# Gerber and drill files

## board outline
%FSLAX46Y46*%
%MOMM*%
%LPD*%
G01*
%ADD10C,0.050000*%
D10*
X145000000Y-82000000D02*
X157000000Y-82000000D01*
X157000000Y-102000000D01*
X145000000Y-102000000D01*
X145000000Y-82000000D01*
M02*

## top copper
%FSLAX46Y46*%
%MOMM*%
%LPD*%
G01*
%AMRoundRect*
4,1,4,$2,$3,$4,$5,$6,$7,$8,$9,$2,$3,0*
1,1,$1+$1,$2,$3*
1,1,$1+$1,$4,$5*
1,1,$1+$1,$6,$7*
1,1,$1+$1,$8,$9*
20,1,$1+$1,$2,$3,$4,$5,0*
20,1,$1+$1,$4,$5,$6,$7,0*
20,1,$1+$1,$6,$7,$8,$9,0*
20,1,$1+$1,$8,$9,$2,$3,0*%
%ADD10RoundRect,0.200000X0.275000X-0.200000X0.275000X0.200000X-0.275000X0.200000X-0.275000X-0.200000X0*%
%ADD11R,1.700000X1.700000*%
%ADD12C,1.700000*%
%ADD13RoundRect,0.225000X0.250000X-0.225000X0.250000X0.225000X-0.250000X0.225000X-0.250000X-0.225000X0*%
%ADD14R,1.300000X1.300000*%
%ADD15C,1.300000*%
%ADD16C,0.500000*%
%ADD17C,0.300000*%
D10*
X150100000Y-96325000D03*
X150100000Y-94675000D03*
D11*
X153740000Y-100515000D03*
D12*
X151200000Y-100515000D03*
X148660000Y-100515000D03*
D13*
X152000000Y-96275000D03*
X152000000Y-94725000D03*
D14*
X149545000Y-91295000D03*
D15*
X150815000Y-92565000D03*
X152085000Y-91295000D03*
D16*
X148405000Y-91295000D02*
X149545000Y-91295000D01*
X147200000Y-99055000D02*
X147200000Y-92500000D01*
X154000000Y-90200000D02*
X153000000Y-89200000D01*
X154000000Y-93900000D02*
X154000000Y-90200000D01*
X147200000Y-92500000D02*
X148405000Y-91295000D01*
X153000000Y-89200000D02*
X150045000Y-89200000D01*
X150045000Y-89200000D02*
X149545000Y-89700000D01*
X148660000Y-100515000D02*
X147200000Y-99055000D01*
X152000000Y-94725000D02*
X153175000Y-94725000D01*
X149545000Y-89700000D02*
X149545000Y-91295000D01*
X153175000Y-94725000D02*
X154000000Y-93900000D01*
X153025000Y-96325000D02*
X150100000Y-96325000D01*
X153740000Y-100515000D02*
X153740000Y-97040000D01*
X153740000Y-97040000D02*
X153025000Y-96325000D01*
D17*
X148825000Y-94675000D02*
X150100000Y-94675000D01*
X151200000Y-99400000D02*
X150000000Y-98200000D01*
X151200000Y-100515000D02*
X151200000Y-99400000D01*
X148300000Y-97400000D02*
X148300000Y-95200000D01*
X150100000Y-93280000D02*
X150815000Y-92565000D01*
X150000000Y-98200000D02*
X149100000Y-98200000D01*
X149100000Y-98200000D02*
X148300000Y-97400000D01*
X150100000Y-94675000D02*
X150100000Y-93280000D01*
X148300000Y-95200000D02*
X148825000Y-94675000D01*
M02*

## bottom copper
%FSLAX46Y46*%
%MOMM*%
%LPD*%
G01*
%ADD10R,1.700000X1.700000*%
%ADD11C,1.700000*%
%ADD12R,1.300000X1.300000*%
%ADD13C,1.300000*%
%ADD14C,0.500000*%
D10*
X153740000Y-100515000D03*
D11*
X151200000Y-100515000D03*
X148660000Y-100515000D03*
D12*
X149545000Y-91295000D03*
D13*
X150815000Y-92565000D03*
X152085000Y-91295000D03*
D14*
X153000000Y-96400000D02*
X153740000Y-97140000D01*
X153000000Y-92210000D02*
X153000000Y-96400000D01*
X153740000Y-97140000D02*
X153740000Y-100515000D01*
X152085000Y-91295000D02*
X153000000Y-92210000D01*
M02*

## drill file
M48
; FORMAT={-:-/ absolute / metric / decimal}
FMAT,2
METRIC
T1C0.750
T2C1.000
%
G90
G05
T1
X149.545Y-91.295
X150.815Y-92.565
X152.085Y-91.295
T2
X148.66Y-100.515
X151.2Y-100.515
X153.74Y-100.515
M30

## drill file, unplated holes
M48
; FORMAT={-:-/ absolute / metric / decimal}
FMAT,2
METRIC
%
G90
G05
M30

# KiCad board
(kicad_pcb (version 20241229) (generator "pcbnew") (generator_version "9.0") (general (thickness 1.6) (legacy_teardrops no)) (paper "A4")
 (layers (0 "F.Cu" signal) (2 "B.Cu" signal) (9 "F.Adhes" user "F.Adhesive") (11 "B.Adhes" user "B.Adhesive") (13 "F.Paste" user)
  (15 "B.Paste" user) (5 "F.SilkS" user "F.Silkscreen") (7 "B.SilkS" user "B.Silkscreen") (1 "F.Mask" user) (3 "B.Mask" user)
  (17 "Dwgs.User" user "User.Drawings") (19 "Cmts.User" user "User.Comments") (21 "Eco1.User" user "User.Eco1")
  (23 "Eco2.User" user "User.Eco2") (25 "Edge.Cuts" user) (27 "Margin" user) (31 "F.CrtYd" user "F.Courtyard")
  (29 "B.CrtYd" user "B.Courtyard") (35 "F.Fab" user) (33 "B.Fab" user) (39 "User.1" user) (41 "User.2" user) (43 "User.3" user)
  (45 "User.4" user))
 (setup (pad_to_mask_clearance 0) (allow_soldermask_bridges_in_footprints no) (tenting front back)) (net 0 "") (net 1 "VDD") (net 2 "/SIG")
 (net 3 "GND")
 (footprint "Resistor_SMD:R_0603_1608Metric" (layer "F.Cu") (at 150.1 95.5 90)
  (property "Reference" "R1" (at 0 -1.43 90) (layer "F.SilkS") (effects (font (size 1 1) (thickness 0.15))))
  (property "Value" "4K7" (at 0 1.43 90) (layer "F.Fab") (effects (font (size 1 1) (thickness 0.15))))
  (pad "1" smd roundrect (at -0.825 0 90) (size 0.8 0.95) (layers "F.Cu" "F.Mask" "F.Paste") (roundrect_rratio 0.25) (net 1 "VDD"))
  (pad "2" smd roundrect (at 0.825 0 90) (size 0.8 0.95) (layers "F.Cu" "F.Mask" "F.Paste") (roundrect_rratio 0.25) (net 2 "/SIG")))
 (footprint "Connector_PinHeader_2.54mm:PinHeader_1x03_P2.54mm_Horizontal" (layer "F.Cu") (at 153.74 100.515 -90)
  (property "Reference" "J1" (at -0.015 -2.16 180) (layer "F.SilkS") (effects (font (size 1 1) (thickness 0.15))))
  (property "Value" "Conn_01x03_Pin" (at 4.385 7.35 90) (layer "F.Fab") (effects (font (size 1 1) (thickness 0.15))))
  (pad "1" thru_hole rect (at 0 0 270) (size 1.7 1.7) (drill 1) (layers "*.Cu" "*.Mask") (remove_unused_layers no) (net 1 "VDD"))
  (pad "2" thru_hole circle (at 0 2.54 270) (size 1.7 1.7) (drill 1) (layers "*.Cu" "*.Mask") (remove_unused_layers no) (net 2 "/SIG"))
  (pad "3" thru_hole circle (at 0 5.08 270) (size 1.7 1.7) (drill 1) (layers "*.Cu" "*.Mask") (remove_unused_layers no) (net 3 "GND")))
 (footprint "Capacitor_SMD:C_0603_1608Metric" (layer "F.Cu") (at 152 95.5 90)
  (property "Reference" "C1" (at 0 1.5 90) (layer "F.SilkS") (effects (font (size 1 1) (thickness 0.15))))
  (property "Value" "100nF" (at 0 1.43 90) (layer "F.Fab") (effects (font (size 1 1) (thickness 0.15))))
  (pad "1" smd roundrect (at -0.775 0 90) (size 0.9 0.95) (layers "F.Cu" "F.Mask" "F.Paste") (roundrect_rratio 0.25) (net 1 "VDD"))
  (pad "2" smd roundrect (at 0.775 0 90) (size 0.9 0.95) (layers "F.Cu" "F.Mask" "F.Paste") (roundrect_rratio 0.25) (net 3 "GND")))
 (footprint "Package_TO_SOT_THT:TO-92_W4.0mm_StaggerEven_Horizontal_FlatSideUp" (layer "F.Cu") (at 149.545 91.295)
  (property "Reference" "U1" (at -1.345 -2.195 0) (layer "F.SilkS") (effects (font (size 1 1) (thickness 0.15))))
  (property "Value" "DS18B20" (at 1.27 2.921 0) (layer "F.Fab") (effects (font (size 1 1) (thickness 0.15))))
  (pad "1" thru_hole rect (at 0 0 270) (size 1.3 1.3) (drill 0.75) (layers "*.Cu" "*.Mask") (remove_unused_layers no) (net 3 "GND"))
  (pad "2" thru_hole circle (at 1.27 1.27 270) (size 1.3 1.3) (drill 0.75) (layers "*.Cu" "*.Mask") (remove_unused_layers no) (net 2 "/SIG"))
  (pad "3" thru_hole circle (at 2.54 0 270) (size 1.3 1.3) (drill 0.75) (layers "*.Cu" "*.Mask") (remove_unused_layers no) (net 1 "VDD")))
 (gr_rect (start 145 82) (end 157 102) (stroke (width 0.05) (type default)) (fill no) (layer "Edge.Cuts"))
 (segment (start 148.405 91.295) (end 149.545 91.295) (width 0.5) (layer "F.Cu") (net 3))
 (segment (start 147.2 99.055) (end 147.2 92.5) (width 0.5) (layer "F.Cu") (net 3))
 (segment (start 154 90.2) (end 153 89.2) (width 0.5) (layer "F.Cu") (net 3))
 (segment (start 154 93.9) (end 154 90.2) (width 0.5) (layer "F.Cu") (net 3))
 (segment (start 147.2 92.5) (end 148.405 91.295) (width 0.5) (layer "F.Cu") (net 3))
 (segment (start 153 89.2) (end 150.045 89.2) (width 0.5) (layer "F.Cu") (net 3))
 (segment (start 150.045 89.2) (end 149.545 89.7) (width 0.5) (layer "F.Cu") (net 3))
 (segment (start 148.66 100.515) (end 147.2 99.055) (width 0.5) (layer "F.Cu") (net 3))
 (segment (start 152 94.725) (end 153.175 94.725) (width 0.5) (layer "F.Cu") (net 3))
 (segment (start 149.545 89.7) (end 149.545 91.295) (width 0.5) (layer "F.Cu") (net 3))
 (segment (start 153.175 94.725) (end 154 93.9) (width 0.5) (layer "F.Cu") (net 3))
 (segment (start 153.025 96.325) (end 150.1 96.325) (width 0.5) (layer "F.Cu") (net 1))
 (segment (start 153.74 100.515) (end 153.74 97.04) (width 0.5) (layer "F.Cu") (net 1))
 (segment (start 153.74 97.04) (end 153.025 96.325) (width 0.5) (layer "F.Cu") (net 1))
 (segment (start 153 96.4) (end 153.74 97.14) (width 0.5) (layer "B.Cu") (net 1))
 (segment (start 153 92.21) (end 153 96.4) (width 0.5) (layer "B.Cu") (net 1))
 (segment (start 153.74 97.14) (end 153.74 100.515) (width 0.5) (layer "B.Cu") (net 1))
 (segment (start 152.085 91.295) (end 153 92.21) (width 0.5) (layer "B.Cu") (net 1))
 (segment (start 148.825 94.675) (end 150.1 94.675) (width 0.3) (layer "F.Cu") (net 2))
 (segment (start 151.2 99.4) (end 150 98.2) (width 0.3) (layer "F.Cu") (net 2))
 (segment (start 151.2 100.515) (end 151.2 99.4) (width 0.3) (layer "F.Cu") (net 2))
 (segment (start 148.3 97.4) (end 148.3 95.2) (width 0.3) (layer "F.Cu") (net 2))
 (segment (start 150.1 93.28) (end 150.815 92.565) (width 0.3) (layer "F.Cu") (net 2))
 (segment (start 150 98.2) (end 149.1 98.2) (width 0.3) (layer "F.Cu") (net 2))
 (segment (start 149.1 98.2) (end 148.3 97.4) (width 0.3) (layer "F.Cu") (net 2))
 (segment (start 150.1 94.675) (end 150.1 93.28) (width 0.3) (layer "F.Cu") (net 2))
 (segment (start 148.3 95.2) (end 148.825 94.675) (width 0.3) (layer "F.Cu") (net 2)))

